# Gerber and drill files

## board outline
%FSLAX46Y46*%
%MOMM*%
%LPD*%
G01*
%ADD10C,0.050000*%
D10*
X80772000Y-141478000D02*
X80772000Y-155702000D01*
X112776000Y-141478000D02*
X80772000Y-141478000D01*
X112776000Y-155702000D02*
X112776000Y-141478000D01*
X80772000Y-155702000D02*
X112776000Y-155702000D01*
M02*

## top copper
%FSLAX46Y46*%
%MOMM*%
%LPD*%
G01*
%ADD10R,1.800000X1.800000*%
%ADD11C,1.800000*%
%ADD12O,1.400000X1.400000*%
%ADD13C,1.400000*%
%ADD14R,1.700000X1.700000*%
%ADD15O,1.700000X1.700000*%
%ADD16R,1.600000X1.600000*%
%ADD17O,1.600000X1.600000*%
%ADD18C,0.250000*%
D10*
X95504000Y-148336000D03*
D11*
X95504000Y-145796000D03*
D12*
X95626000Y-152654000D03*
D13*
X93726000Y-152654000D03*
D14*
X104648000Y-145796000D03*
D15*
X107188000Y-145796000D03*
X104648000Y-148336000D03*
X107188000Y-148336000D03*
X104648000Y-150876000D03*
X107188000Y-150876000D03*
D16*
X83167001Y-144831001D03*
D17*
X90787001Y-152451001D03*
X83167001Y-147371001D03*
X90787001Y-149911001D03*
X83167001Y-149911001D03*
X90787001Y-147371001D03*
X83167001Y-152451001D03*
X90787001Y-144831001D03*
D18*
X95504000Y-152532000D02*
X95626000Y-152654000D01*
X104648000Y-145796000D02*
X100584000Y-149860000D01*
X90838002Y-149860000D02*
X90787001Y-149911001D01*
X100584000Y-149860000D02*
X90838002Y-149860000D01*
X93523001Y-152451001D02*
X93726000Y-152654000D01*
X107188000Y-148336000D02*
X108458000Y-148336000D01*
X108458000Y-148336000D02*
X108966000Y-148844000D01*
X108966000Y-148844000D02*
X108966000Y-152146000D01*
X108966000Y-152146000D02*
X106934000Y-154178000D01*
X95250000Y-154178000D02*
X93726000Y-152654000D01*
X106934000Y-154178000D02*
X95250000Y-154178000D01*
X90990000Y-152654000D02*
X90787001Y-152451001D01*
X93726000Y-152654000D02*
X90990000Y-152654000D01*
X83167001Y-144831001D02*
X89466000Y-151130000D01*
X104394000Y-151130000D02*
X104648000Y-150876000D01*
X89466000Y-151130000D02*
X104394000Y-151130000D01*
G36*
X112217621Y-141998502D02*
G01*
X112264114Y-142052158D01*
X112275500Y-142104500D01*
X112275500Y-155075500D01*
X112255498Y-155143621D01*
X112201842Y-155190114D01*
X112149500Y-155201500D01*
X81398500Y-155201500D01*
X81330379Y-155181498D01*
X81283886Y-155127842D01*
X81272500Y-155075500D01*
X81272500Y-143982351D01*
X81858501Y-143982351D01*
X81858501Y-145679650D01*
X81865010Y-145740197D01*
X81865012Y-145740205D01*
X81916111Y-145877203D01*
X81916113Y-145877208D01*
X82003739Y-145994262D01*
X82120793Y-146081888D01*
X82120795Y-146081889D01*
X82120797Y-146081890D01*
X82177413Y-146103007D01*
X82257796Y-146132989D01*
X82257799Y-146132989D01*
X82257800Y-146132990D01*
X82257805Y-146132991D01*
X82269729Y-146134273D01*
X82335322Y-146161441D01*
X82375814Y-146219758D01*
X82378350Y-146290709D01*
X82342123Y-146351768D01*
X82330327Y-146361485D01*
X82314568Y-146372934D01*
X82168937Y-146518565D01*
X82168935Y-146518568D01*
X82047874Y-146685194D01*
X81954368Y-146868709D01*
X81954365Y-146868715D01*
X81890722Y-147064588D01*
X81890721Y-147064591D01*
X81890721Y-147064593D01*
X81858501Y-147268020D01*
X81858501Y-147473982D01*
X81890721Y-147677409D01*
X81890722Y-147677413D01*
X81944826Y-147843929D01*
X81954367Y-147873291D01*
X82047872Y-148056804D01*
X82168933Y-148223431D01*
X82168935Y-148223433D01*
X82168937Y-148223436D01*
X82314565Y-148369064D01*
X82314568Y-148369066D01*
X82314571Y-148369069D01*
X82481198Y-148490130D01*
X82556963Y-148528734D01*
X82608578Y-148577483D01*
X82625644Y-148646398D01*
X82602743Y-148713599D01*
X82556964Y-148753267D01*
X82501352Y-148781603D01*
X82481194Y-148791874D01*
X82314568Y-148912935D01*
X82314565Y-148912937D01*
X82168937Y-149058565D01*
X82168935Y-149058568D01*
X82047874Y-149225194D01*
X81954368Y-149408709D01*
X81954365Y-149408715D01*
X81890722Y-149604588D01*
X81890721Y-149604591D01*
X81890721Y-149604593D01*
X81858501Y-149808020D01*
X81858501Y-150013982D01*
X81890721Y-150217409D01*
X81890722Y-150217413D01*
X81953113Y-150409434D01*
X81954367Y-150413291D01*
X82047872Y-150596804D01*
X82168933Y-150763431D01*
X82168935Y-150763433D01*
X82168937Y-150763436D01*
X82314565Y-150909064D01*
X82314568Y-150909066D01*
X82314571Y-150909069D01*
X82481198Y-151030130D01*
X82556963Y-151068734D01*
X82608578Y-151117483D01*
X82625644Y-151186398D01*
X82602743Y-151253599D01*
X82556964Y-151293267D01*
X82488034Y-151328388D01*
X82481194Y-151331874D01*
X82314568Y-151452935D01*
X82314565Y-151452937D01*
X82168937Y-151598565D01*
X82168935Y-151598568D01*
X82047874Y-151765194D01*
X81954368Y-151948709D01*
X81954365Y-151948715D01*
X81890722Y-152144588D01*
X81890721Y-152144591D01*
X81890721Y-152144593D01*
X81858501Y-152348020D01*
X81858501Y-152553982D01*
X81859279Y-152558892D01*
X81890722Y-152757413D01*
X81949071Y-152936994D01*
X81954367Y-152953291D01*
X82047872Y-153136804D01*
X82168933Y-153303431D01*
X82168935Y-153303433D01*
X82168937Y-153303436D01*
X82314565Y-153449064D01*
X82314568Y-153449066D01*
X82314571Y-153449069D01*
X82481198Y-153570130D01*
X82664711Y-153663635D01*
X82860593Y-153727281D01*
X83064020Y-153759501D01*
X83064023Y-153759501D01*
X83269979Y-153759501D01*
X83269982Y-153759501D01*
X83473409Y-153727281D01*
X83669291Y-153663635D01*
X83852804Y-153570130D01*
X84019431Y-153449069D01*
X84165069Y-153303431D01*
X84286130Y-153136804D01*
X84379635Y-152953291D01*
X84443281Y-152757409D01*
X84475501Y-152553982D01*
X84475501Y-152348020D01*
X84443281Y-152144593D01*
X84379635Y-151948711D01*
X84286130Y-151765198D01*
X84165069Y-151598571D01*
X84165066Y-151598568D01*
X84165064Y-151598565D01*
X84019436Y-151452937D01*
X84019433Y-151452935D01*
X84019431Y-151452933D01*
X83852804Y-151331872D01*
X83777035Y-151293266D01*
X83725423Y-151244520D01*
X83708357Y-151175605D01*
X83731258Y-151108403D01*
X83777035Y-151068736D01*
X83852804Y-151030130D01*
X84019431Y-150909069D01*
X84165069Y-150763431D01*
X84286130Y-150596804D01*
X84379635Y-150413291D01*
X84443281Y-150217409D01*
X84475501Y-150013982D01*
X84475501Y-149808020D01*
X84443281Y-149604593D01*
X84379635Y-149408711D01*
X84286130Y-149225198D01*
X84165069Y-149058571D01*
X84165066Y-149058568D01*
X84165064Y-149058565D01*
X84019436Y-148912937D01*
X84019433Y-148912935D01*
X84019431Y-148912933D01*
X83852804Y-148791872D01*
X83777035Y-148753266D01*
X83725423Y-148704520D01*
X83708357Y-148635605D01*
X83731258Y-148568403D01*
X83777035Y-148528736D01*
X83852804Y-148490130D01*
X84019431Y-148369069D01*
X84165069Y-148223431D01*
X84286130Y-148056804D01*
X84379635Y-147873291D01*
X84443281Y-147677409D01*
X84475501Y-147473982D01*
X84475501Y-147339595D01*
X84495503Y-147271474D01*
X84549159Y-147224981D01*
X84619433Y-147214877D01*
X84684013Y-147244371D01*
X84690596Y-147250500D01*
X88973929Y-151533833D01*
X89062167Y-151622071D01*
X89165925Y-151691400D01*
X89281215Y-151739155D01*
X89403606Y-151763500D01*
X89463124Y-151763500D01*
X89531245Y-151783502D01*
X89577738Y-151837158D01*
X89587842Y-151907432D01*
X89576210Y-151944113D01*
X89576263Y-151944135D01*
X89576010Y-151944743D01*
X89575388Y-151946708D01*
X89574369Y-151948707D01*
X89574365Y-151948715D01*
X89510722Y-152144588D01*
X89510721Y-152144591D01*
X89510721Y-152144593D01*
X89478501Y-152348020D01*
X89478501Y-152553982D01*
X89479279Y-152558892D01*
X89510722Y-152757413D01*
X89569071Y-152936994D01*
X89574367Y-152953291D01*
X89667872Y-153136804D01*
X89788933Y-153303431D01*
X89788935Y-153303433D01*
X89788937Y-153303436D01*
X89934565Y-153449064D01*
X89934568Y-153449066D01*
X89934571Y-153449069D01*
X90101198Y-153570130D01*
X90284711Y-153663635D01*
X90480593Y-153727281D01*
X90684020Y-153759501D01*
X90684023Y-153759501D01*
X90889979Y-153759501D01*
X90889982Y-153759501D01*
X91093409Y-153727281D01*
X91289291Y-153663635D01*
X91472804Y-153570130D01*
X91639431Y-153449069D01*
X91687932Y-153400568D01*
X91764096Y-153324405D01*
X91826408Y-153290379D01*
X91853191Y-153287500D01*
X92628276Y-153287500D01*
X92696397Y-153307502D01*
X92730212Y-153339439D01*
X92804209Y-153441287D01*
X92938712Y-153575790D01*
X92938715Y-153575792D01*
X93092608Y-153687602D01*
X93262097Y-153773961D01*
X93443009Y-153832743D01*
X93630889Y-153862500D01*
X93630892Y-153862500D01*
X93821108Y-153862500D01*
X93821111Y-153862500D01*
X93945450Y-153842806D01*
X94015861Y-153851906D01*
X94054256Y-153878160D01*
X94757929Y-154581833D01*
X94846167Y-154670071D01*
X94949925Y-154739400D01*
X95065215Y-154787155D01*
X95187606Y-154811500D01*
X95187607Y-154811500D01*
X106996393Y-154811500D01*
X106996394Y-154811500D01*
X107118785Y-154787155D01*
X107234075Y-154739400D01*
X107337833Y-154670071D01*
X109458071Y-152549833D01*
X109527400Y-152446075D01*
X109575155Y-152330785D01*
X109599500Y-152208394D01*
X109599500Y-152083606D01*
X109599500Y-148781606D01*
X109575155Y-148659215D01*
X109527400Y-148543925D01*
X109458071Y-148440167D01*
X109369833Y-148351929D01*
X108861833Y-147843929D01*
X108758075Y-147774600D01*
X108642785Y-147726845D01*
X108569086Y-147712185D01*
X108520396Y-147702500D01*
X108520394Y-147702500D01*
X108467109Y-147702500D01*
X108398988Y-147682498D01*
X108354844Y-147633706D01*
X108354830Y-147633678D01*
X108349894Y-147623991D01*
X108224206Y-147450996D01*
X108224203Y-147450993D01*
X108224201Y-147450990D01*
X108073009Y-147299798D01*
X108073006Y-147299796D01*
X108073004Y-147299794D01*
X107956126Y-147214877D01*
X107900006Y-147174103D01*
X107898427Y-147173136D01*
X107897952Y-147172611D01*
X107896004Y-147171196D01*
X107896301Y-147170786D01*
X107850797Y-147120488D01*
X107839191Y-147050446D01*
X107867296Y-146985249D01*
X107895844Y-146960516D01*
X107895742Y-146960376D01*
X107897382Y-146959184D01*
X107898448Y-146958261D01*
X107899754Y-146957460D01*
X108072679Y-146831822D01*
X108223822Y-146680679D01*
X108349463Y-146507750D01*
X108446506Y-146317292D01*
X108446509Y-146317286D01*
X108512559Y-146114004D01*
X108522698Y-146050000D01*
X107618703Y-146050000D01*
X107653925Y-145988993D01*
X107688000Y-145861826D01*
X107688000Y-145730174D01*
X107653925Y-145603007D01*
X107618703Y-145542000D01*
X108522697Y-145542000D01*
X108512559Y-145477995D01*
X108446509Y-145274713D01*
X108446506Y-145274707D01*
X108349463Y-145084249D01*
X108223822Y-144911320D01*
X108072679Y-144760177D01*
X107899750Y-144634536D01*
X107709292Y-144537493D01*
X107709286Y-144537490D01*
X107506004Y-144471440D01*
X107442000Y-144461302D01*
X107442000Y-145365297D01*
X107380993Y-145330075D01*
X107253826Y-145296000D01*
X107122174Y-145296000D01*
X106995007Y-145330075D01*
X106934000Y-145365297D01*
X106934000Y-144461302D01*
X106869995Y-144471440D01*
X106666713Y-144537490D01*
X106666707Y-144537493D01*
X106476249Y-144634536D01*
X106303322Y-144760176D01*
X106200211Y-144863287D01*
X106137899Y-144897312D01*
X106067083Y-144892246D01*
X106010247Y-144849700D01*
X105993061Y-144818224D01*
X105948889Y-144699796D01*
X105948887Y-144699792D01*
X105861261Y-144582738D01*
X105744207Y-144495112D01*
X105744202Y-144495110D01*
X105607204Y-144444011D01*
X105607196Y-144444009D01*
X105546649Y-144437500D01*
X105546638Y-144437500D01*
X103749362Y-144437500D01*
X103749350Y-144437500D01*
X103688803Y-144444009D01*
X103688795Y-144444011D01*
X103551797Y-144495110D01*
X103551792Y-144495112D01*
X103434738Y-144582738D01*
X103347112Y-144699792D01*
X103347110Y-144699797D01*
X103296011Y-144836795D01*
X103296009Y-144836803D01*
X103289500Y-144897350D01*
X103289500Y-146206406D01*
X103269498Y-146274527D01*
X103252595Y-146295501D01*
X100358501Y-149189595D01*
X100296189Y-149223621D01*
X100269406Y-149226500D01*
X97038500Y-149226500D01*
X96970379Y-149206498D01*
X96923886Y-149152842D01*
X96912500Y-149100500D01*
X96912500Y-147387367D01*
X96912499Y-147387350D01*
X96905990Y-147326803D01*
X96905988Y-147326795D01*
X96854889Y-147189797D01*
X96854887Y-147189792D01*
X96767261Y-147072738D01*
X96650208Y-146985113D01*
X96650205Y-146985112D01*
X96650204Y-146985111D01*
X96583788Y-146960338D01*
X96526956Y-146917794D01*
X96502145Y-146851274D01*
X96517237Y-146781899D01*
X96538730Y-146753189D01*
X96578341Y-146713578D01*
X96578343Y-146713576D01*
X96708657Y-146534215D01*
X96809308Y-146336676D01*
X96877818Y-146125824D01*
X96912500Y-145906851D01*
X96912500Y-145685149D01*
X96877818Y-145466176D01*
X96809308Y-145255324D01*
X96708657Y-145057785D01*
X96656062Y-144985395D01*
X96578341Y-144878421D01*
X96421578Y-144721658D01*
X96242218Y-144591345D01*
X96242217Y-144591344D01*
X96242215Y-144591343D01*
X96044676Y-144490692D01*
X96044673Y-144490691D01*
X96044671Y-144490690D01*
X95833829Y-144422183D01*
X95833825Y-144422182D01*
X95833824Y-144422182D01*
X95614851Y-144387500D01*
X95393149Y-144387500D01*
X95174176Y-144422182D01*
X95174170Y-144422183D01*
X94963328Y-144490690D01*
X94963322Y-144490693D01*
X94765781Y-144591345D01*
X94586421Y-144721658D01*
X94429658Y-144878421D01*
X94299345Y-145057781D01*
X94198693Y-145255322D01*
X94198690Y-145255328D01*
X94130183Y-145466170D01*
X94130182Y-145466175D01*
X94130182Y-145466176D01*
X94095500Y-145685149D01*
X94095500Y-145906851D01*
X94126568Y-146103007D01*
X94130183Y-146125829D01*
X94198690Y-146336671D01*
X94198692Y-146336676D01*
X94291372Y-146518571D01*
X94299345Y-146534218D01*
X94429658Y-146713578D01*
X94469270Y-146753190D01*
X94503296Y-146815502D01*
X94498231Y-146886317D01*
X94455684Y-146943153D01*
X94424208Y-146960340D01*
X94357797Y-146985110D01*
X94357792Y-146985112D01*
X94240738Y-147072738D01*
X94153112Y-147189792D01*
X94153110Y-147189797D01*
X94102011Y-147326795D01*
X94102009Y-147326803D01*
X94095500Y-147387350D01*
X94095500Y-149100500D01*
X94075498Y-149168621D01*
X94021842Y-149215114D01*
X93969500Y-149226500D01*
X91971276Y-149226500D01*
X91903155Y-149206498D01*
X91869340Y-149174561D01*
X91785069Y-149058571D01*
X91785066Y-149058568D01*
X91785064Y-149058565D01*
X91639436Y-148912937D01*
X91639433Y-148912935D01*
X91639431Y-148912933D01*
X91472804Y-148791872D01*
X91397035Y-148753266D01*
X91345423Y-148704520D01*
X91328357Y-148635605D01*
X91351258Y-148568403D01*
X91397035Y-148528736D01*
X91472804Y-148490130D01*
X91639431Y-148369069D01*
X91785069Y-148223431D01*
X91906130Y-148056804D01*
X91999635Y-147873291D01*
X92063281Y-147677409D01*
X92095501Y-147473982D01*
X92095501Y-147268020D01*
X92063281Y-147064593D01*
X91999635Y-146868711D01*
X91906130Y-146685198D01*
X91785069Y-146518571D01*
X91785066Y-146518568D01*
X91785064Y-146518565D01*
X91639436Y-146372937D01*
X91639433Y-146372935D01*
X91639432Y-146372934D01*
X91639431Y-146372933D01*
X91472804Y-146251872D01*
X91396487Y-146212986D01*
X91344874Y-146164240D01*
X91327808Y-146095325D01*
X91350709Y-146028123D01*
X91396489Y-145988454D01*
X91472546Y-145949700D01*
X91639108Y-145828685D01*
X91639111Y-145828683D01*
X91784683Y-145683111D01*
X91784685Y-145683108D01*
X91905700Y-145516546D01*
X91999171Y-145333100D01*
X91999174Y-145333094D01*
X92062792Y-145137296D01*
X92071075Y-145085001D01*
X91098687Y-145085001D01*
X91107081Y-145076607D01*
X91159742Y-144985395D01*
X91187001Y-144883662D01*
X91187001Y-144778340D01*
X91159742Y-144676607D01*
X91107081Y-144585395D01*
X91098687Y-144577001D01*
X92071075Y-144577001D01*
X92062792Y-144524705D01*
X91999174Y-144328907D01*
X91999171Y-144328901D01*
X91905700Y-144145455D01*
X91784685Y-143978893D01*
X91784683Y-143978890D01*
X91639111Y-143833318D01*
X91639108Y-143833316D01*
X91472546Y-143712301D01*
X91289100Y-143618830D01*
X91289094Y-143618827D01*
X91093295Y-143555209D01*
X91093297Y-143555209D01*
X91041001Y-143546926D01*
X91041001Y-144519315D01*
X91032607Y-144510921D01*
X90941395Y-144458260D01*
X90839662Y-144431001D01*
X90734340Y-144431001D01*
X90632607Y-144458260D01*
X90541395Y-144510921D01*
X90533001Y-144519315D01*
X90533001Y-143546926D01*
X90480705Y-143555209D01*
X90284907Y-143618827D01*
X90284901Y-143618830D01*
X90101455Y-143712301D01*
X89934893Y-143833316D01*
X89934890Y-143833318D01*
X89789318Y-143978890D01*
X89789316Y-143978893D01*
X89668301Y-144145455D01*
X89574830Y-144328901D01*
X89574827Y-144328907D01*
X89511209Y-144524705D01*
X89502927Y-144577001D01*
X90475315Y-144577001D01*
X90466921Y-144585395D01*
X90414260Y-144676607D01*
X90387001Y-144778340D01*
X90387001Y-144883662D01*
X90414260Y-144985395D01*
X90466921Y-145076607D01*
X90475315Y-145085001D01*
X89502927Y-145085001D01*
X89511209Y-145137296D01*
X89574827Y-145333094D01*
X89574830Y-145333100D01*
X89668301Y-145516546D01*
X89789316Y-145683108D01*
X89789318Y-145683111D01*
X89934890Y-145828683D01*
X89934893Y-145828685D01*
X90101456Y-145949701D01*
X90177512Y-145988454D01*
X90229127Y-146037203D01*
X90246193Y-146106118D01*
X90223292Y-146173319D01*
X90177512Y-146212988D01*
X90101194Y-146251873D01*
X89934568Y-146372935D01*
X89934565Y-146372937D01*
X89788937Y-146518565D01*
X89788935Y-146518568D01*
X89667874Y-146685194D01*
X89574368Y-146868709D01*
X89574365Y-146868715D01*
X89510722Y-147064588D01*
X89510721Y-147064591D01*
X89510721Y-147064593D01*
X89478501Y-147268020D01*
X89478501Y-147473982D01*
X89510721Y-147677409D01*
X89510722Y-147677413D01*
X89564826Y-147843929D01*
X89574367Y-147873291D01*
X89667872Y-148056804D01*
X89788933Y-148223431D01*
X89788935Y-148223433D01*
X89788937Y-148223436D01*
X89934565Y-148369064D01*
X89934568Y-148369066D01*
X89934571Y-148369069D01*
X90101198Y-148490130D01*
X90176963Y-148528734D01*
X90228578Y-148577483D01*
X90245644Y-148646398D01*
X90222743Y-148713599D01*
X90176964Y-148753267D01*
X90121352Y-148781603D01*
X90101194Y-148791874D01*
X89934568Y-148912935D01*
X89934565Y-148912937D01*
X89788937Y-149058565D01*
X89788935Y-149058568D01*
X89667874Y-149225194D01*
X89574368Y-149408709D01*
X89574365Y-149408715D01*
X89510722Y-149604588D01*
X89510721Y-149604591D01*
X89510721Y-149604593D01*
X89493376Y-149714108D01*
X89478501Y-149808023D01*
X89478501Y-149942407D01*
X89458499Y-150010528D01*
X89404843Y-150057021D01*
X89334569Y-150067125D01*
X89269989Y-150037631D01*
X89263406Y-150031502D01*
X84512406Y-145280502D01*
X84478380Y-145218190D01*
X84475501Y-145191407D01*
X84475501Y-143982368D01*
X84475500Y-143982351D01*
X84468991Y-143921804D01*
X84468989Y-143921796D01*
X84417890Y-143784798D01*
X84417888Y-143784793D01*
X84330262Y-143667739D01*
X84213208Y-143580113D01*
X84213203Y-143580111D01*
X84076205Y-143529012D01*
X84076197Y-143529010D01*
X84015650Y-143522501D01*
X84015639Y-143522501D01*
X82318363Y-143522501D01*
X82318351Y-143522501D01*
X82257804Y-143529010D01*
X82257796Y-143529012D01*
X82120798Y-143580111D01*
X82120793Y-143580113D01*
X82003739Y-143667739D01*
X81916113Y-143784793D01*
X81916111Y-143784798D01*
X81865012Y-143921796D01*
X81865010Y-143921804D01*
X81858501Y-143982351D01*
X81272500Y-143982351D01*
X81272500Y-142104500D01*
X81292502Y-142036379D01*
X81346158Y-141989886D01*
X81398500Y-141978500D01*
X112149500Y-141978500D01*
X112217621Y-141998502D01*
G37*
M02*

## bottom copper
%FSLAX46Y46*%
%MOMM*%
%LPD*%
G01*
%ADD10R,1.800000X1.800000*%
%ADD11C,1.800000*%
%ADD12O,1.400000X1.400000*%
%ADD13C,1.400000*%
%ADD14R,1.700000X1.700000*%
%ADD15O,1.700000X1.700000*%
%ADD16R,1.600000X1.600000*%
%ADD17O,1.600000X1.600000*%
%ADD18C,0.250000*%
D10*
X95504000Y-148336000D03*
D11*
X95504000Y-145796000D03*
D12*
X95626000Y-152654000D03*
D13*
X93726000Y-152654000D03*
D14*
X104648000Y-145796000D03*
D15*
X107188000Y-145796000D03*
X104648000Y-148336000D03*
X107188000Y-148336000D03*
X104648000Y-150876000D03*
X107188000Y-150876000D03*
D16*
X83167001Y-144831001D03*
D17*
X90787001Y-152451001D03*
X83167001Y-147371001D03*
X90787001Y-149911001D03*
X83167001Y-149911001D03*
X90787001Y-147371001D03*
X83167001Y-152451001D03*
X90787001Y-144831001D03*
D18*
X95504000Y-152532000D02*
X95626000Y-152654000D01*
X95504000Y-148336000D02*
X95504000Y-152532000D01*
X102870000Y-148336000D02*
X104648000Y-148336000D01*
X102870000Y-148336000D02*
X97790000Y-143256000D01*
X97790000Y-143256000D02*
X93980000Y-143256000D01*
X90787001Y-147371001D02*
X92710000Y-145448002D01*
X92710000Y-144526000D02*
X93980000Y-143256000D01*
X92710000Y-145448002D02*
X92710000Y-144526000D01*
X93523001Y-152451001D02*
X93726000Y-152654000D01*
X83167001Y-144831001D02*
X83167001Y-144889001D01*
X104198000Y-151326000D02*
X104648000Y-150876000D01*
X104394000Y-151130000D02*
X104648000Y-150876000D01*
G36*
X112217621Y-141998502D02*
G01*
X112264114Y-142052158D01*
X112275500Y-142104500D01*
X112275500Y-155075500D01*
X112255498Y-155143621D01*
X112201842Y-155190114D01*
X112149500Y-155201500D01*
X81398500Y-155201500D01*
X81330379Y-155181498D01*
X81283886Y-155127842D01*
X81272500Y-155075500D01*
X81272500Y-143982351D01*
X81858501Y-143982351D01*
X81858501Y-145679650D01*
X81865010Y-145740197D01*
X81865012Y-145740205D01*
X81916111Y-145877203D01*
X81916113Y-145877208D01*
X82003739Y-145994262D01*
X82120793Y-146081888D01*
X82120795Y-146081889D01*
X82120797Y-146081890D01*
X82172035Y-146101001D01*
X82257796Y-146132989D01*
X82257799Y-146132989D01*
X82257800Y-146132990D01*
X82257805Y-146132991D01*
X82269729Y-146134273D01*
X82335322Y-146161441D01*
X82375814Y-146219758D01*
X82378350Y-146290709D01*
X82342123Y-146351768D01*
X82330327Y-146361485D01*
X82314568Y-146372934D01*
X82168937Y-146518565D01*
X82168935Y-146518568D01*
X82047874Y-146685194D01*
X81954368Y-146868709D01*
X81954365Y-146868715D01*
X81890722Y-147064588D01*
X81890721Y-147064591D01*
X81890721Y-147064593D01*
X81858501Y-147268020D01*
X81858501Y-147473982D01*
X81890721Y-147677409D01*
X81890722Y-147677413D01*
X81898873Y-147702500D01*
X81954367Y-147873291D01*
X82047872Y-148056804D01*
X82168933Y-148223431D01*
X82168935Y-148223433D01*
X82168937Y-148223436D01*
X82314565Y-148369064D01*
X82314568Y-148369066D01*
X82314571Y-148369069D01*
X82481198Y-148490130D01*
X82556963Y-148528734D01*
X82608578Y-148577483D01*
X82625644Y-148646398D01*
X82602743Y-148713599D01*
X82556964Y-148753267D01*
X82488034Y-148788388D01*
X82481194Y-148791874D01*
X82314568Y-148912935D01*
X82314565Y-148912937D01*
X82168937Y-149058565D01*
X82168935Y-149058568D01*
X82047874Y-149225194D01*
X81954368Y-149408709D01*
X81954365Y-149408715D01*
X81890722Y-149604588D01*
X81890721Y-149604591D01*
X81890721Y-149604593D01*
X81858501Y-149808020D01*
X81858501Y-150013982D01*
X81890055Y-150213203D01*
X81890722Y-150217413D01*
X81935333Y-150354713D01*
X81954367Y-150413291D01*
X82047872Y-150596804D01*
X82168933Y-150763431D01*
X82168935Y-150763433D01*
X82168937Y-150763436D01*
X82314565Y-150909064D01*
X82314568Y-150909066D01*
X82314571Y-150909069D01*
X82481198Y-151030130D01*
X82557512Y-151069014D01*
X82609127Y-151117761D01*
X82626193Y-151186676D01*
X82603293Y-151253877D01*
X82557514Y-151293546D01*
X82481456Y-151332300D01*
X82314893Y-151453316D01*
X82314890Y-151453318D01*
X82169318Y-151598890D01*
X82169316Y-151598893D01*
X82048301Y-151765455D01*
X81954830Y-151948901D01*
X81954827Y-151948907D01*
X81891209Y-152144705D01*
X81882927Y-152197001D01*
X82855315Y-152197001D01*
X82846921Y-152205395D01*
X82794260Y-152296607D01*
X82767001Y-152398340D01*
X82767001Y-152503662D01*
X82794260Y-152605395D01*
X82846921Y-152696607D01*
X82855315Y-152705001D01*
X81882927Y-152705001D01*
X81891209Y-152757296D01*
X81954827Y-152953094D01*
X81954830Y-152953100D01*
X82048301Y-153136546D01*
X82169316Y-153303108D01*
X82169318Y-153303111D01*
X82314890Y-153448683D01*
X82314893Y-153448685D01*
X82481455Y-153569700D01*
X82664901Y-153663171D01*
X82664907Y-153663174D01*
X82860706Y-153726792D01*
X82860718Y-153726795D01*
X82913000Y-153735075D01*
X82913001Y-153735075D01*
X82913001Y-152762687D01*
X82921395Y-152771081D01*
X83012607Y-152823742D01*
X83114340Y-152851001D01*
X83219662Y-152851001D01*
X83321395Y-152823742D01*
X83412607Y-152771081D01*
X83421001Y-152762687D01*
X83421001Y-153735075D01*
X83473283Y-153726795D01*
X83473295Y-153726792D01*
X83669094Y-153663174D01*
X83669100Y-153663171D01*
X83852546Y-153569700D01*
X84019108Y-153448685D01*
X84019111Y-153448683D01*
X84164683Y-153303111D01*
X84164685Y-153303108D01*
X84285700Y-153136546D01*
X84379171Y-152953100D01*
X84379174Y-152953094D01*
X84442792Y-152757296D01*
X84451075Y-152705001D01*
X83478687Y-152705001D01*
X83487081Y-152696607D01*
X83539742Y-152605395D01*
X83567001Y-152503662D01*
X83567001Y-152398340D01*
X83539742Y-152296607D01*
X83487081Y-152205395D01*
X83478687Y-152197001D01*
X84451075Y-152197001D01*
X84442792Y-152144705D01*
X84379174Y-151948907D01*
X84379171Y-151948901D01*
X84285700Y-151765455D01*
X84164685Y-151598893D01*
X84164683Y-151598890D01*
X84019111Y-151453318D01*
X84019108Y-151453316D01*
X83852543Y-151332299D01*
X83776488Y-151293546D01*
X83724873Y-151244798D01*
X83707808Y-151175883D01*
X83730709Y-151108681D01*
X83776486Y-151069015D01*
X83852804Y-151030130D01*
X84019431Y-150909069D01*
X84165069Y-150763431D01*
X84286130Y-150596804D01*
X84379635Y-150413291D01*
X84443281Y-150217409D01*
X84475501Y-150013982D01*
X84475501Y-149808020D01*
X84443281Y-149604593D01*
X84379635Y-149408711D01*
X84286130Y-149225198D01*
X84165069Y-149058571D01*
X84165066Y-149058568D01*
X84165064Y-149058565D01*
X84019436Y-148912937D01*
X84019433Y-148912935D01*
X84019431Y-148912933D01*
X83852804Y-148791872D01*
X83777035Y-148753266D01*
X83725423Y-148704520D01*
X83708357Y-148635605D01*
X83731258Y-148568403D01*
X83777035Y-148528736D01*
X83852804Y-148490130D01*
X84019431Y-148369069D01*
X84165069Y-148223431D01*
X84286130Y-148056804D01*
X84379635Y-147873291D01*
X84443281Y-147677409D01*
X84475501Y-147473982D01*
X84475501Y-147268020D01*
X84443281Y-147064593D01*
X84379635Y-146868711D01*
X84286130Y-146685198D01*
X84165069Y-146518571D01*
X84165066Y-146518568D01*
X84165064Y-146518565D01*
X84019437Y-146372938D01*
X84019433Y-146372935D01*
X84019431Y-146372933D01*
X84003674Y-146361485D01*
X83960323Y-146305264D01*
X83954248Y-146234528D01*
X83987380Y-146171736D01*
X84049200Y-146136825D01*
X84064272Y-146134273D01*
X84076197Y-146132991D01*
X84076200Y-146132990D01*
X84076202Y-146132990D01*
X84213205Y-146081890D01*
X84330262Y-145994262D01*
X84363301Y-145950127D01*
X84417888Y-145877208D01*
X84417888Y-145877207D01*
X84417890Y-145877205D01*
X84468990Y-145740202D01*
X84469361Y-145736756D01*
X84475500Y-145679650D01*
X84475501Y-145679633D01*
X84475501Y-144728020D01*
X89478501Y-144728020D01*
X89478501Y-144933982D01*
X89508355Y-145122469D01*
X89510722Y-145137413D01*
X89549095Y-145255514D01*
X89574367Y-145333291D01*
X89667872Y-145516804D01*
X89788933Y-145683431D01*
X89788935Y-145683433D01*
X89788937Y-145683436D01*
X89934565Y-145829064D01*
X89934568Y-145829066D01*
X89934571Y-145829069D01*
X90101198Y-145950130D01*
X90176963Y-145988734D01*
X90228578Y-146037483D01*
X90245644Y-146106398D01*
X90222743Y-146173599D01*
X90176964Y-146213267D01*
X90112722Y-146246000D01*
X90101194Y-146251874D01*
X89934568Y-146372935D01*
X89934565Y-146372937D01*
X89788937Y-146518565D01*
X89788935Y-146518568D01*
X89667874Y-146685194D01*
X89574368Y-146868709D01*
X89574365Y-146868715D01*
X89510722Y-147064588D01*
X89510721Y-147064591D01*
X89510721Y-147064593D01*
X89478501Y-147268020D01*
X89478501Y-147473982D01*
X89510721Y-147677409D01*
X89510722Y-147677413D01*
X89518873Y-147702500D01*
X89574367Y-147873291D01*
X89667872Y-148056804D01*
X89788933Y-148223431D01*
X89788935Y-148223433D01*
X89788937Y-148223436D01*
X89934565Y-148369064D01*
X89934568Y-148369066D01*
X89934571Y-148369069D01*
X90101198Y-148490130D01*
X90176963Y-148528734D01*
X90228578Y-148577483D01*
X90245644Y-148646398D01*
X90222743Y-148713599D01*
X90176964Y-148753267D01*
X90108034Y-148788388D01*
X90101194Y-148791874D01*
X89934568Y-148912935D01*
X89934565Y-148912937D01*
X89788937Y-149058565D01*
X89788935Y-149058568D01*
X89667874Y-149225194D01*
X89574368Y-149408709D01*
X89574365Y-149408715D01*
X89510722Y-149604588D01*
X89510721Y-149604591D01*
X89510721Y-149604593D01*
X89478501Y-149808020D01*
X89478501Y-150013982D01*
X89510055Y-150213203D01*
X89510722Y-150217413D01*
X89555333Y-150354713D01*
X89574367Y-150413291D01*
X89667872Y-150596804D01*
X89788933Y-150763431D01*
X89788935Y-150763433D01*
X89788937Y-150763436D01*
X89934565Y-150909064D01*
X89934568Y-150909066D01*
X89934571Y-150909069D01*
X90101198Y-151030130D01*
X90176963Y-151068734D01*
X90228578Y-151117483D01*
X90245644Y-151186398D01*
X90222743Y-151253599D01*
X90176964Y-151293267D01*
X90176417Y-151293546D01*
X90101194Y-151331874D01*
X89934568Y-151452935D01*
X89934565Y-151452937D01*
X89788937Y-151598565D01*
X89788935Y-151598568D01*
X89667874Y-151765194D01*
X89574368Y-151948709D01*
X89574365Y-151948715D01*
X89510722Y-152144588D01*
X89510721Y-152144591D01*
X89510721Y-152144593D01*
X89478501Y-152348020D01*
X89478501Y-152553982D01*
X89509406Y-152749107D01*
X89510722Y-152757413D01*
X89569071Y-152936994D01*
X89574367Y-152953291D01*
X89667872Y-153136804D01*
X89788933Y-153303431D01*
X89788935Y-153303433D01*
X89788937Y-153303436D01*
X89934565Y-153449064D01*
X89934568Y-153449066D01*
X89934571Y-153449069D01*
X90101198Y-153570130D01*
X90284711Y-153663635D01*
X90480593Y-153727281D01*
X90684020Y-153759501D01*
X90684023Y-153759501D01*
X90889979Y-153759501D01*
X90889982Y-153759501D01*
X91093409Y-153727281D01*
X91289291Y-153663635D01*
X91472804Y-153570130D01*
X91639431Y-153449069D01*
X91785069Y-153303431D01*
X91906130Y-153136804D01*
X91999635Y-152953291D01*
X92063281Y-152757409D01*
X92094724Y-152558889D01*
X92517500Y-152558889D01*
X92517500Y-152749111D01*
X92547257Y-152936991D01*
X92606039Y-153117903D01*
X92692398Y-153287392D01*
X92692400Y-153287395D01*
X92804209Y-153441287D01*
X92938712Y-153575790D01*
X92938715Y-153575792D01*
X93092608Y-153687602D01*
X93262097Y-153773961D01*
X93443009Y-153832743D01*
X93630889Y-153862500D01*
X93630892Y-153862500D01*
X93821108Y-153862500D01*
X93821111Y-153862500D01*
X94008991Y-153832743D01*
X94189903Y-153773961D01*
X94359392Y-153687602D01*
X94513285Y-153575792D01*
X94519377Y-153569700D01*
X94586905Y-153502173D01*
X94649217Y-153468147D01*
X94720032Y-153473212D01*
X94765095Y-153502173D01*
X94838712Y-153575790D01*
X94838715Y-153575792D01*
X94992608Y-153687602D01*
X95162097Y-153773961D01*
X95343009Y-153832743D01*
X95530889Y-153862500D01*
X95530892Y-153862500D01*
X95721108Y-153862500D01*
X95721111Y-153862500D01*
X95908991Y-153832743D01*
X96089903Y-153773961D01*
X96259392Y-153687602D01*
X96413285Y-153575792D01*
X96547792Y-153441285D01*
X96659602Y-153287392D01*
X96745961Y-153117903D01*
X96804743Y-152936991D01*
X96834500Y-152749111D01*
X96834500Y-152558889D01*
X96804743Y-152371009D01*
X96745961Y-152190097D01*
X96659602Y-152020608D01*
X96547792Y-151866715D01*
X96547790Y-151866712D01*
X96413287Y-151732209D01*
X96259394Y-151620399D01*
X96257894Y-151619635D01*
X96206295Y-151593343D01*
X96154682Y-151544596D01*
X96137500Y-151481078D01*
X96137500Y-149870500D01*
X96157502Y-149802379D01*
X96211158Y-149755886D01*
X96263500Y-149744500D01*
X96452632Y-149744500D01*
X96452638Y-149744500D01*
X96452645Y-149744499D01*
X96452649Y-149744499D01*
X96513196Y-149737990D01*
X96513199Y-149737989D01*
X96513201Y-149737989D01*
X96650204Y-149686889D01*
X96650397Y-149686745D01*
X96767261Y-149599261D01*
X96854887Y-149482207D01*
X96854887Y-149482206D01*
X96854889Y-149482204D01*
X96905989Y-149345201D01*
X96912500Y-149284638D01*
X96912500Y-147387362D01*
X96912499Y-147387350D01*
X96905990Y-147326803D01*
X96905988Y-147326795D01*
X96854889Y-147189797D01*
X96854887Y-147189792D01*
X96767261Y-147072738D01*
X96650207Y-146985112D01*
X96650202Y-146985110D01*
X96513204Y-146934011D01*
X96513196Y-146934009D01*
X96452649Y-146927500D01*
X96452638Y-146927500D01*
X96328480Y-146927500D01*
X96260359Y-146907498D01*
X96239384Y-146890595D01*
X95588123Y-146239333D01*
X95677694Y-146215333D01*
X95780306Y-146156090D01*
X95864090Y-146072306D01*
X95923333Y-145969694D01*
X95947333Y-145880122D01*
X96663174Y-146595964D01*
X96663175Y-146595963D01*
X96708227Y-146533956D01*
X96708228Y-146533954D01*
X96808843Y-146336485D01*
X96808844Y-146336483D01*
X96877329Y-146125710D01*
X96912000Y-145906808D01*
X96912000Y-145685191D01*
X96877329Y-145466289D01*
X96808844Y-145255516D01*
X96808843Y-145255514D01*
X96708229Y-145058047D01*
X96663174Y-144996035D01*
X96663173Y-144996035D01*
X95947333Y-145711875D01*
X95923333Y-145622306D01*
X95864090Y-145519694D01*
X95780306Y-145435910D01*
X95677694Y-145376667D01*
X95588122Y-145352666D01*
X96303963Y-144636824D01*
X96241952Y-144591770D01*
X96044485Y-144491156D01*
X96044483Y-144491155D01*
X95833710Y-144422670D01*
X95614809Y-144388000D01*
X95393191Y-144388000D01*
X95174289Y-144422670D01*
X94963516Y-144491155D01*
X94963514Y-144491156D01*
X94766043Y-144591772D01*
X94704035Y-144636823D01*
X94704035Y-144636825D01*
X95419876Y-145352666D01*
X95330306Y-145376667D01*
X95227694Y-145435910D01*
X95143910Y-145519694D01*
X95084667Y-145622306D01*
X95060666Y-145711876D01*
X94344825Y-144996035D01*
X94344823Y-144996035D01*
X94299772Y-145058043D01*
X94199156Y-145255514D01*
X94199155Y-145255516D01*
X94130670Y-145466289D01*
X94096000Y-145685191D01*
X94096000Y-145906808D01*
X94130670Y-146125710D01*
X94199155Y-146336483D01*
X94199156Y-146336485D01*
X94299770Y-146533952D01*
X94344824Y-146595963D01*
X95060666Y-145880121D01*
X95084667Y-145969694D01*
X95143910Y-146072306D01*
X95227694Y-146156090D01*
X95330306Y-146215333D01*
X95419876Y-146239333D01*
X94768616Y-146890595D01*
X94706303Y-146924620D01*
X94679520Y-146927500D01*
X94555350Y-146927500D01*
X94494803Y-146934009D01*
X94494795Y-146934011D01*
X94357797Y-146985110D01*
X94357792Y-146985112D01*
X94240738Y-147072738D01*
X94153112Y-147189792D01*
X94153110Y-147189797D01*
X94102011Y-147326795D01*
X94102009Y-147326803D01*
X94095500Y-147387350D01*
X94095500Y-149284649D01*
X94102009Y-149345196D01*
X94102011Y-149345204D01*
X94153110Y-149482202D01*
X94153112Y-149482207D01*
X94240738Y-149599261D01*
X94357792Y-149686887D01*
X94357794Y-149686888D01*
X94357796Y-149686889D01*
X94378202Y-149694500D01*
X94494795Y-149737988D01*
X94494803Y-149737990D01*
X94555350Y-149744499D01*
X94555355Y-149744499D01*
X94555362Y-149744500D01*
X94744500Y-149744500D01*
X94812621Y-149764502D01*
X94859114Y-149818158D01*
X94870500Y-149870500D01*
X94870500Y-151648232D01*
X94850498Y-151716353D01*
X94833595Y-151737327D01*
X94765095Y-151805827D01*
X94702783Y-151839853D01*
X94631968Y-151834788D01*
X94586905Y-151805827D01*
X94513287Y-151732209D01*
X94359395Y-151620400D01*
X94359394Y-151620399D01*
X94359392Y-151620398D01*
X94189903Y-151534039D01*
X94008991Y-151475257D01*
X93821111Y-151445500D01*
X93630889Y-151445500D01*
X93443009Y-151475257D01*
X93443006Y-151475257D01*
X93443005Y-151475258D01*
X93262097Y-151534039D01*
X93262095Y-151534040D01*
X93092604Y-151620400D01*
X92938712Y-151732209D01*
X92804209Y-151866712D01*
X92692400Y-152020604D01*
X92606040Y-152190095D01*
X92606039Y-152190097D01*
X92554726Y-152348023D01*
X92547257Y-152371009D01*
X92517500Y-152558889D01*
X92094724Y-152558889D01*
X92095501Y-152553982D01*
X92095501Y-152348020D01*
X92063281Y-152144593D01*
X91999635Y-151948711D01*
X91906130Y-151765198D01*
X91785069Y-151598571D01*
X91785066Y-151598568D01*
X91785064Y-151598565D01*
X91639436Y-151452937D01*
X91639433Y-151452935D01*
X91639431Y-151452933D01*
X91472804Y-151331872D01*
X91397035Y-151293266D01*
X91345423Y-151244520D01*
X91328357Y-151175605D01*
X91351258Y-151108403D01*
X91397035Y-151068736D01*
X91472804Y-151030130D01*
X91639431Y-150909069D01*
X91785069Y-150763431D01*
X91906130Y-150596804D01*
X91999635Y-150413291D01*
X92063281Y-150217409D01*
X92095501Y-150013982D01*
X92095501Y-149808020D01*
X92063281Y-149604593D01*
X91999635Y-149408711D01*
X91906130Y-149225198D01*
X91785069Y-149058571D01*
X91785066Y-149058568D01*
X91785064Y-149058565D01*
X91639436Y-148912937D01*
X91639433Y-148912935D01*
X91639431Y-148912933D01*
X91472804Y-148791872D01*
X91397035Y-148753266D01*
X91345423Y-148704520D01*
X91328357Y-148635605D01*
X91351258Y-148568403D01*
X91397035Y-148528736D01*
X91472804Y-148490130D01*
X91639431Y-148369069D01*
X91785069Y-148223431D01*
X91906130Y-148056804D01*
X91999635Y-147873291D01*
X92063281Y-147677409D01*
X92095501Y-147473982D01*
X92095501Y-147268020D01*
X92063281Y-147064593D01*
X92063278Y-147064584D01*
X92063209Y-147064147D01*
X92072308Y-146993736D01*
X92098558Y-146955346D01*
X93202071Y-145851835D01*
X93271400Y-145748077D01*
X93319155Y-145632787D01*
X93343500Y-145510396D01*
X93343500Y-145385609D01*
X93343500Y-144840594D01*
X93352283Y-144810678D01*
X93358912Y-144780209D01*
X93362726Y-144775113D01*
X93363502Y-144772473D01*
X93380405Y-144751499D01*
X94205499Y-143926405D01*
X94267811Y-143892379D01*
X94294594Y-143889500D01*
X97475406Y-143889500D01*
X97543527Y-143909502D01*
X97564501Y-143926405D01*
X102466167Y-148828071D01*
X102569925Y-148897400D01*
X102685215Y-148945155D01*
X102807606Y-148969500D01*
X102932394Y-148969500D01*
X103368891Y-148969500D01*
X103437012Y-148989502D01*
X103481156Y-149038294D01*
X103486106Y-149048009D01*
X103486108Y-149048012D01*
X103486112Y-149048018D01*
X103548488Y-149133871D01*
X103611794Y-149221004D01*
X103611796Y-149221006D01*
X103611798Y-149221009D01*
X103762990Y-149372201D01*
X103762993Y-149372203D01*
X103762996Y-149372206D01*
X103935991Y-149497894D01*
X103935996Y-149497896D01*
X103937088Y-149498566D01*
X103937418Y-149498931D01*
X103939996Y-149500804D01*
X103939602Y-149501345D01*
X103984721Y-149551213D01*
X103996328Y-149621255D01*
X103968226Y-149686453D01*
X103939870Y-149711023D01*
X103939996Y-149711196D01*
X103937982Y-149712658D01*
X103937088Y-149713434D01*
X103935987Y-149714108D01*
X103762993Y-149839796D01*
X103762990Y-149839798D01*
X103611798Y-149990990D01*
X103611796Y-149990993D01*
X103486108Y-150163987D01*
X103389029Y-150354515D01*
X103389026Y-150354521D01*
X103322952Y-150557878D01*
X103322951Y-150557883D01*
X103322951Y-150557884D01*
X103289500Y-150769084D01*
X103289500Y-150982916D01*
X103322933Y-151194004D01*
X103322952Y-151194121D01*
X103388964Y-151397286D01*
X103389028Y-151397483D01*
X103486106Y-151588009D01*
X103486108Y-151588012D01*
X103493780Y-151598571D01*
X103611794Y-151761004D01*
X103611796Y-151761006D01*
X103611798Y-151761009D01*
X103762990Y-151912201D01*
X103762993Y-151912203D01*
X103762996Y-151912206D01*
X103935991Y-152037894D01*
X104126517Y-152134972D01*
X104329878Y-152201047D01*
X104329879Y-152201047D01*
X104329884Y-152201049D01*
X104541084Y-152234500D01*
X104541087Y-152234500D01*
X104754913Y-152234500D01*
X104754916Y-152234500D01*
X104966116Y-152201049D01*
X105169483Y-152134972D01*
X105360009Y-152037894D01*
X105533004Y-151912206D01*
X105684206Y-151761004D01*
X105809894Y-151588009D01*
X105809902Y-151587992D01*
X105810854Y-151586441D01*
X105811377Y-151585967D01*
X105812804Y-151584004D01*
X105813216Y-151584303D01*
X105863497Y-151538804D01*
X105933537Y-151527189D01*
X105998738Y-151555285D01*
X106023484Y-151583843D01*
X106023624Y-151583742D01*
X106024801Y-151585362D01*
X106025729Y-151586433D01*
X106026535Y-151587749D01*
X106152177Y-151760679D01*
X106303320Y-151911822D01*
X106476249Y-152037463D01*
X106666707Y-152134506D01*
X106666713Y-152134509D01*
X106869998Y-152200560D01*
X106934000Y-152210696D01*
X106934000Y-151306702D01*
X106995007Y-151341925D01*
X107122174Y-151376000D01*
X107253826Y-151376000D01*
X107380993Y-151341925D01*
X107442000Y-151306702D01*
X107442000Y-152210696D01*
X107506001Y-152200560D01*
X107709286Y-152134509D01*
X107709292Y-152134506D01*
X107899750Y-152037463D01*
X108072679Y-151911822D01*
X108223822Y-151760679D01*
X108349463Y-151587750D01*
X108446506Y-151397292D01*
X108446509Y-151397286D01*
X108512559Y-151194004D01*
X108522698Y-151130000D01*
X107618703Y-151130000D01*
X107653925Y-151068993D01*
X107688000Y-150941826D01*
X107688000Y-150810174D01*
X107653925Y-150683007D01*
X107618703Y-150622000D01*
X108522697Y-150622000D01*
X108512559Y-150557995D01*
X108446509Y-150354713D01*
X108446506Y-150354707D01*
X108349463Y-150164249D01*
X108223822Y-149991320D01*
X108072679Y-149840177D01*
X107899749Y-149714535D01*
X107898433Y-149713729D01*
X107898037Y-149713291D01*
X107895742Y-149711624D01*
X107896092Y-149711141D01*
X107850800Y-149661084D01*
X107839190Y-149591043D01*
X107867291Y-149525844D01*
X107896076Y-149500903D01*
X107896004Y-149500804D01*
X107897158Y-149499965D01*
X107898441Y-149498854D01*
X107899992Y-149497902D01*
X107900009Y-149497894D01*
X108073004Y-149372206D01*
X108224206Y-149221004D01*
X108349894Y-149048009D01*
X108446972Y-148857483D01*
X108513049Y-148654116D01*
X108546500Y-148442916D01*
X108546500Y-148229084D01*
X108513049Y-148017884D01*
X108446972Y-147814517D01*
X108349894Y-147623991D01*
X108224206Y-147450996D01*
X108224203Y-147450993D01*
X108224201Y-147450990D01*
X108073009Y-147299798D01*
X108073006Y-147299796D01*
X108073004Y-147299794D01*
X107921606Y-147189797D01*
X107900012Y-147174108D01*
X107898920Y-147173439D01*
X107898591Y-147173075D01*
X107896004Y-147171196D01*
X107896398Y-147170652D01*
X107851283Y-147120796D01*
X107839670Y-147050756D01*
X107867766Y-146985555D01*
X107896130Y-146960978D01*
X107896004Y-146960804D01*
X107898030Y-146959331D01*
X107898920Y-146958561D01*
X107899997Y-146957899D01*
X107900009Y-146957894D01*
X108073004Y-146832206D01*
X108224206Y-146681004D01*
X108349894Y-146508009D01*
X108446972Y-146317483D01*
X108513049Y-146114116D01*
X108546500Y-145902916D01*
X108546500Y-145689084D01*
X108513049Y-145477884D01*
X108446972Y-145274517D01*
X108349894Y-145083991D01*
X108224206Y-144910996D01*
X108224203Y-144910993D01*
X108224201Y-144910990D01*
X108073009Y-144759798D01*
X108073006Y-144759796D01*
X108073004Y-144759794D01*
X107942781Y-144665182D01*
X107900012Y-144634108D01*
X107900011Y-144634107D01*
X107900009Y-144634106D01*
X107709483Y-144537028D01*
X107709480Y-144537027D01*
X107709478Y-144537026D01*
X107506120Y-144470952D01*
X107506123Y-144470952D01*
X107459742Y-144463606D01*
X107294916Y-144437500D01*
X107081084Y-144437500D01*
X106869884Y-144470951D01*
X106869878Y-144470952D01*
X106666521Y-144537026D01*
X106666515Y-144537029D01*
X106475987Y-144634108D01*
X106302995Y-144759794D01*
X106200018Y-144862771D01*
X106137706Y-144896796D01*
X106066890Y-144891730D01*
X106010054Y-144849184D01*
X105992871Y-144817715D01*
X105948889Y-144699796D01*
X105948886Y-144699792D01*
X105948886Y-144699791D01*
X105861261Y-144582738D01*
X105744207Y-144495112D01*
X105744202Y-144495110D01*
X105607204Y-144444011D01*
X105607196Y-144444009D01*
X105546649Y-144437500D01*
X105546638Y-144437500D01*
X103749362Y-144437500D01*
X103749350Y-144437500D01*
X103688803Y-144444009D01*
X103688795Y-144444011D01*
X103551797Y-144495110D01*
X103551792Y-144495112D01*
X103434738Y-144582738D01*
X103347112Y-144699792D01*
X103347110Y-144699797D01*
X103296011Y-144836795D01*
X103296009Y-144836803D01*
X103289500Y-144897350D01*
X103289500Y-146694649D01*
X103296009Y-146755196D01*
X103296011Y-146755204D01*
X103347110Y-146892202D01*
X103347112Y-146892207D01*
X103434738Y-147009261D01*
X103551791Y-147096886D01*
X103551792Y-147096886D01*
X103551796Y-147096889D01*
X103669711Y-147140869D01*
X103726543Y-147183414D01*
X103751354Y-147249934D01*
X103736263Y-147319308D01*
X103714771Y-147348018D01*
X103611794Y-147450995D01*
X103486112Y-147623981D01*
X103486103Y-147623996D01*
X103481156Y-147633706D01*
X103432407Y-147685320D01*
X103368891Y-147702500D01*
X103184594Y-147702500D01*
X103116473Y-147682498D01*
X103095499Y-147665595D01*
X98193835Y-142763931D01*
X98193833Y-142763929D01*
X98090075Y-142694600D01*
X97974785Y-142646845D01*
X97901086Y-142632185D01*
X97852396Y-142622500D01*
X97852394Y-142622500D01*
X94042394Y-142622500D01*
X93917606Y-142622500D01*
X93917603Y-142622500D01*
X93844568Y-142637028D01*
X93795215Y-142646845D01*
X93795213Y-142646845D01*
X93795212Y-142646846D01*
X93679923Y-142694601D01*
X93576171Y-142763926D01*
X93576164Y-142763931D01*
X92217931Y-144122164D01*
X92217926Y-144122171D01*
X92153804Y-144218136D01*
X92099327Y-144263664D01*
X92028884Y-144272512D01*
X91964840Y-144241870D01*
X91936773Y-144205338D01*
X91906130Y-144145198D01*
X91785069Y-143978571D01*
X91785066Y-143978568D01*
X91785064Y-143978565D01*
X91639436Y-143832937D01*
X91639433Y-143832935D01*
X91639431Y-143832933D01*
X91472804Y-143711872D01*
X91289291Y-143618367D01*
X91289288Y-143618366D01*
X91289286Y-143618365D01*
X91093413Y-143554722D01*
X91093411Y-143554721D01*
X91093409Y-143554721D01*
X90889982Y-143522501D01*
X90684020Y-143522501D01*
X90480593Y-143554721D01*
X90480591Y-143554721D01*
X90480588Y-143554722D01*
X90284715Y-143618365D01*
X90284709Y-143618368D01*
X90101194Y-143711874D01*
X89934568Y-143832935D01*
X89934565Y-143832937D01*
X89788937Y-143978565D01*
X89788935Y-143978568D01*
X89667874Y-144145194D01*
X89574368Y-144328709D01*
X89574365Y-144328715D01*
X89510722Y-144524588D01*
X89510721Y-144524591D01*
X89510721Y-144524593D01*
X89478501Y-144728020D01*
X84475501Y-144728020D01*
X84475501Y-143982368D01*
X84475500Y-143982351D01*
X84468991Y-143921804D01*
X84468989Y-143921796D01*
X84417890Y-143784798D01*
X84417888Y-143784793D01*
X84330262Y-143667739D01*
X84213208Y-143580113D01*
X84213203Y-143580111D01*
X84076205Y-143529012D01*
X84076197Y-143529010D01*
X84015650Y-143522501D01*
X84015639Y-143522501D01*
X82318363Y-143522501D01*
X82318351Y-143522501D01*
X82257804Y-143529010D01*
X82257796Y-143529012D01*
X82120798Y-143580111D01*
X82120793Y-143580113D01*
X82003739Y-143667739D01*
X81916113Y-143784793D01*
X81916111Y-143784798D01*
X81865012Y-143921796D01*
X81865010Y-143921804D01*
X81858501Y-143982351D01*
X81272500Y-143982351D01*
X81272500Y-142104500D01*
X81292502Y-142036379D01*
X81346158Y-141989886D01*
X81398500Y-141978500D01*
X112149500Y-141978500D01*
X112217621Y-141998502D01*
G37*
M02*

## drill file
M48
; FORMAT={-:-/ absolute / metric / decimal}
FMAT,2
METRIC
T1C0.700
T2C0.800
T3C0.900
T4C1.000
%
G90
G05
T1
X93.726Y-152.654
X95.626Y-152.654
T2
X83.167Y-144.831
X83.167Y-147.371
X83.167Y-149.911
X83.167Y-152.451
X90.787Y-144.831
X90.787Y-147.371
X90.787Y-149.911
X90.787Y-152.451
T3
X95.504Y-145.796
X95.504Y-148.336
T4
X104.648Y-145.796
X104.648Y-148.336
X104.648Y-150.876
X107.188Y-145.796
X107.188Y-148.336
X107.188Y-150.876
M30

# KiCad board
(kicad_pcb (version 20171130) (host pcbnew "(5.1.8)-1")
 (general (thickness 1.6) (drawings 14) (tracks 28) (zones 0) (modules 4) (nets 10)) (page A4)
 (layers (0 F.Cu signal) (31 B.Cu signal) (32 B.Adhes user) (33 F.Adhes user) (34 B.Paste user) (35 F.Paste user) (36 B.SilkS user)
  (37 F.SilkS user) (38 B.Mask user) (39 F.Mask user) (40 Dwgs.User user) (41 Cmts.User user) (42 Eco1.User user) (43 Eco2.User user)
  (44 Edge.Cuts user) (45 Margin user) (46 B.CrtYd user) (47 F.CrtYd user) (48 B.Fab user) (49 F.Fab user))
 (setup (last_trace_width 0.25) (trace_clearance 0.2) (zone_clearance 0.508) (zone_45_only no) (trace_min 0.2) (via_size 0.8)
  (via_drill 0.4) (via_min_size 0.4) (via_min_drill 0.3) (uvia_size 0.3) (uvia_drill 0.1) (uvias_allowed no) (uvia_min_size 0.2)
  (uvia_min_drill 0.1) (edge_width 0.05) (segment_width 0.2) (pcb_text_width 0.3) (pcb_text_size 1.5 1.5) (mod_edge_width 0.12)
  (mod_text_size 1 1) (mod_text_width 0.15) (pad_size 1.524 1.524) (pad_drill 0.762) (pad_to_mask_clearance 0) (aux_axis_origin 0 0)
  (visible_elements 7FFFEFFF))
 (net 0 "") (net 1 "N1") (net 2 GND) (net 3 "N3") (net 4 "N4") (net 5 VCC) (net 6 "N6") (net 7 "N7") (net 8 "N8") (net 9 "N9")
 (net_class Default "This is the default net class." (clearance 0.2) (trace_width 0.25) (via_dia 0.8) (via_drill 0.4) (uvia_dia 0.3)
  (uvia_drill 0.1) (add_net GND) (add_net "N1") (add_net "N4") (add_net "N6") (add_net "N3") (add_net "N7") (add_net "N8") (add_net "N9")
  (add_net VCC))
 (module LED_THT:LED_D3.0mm (layer F.Cu) (at 95.504 148.336 90)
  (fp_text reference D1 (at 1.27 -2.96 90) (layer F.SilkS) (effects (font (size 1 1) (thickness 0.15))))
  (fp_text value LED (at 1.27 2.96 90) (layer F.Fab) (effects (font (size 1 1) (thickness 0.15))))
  (pad 1 thru_hole rect (at 0 0 90) (size 1.8 1.8) (drill 0.9) (layers *.Cu *.Mask) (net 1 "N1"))
  (pad 2 thru_hole circle (at 2.54 0 90) (size 1.8 1.8) (drill 0.9) (layers *.Cu *.Mask) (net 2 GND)))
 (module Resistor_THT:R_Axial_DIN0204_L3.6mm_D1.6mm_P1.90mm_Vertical (layer F.Cu) (at 93.726 152.654)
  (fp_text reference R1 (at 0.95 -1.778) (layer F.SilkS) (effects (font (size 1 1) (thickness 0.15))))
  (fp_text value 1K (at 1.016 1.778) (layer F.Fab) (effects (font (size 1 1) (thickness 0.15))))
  (pad 2 thru_hole oval (at 1.9 0) (size 1.4 1.4) (drill 0.7) (layers *.Cu *.Mask) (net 1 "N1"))
  (pad 1 thru_hole circle (at 0 0) (size 1.4 1.4) (drill 0.7) (layers *.Cu *.Mask) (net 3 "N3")))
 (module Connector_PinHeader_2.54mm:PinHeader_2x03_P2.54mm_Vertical (layer F.Cu) (at 104.648 145.796)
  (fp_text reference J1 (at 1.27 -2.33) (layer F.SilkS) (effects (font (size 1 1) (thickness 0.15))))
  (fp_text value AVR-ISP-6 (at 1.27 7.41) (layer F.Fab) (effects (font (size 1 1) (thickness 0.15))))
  (pad 1 thru_hole rect (at 0 0) (size 1.7 1.7) (drill 1) (layers *.Cu *.Mask) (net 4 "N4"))
  (pad 2 thru_hole oval (at 2.54 0) (size 1.7 1.7) (drill 1) (layers *.Cu *.Mask) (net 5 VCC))
  (pad 3 thru_hole oval (at 0 2.54) (size 1.7 1.7) (drill 1) (layers *.Cu *.Mask) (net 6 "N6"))
  (pad 4 thru_hole oval (at 2.54 2.54) (size 1.7 1.7) (drill 1) (layers *.Cu *.Mask) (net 3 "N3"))
  (pad 5 thru_hole oval (at 0 5.08) (size 1.7 1.7) (drill 1) (layers *.Cu *.Mask) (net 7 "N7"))
  (pad 6 thru_hole oval (at 2.54 5.08) (size 1.7 1.7) (drill 1) (layers *.Cu *.Mask) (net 2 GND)))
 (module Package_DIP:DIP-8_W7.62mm (layer F.Cu) (at 83.167001 144.831001)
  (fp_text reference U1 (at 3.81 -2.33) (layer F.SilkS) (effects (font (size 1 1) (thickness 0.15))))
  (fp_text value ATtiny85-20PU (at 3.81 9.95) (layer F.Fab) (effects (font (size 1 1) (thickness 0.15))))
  (pad 1 thru_hole rect (at 0 0) (size 1.6 1.6) (drill 0.8) (layers *.Cu *.Mask) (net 7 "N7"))
  (pad 5 thru_hole oval (at 7.62 7.62) (size 1.6 1.6) (drill 0.8) (layers *.Cu *.Mask) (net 3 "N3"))
  (pad 2 thru_hole oval (at 0 2.54) (size 1.6 1.6) (drill 0.8) (layers *.Cu *.Mask) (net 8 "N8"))
  (pad 6 thru_hole oval (at 7.62 5.08) (size 1.6 1.6) (drill 0.8) (layers *.Cu *.Mask) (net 4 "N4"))
  (pad 3 thru_hole oval (at 0 5.08) (size 1.6 1.6) (drill 0.8) (layers *.Cu *.Mask) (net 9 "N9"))
  (pad 7 thru_hole oval (at 7.62 2.54) (size 1.6 1.6) (drill 0.8) (layers *.Cu *.Mask) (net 6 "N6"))
  (pad 4 thru_hole oval (at 0 7.62) (size 1.6 1.6) (drill 0.8) (layers *.Cu *.Mask) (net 2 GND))
  (pad 8 thru_hole oval (at 7.62 0) (size 1.6 1.6) (drill 0.8) (layers *.Cu *.Mask) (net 5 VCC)))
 (gr_line (start 80.772 141.478) (end 80.772 155.702) (layer Edge.Cuts) (width 0.05))
 (gr_line (start 112.776 141.478) (end 80.772 141.478) (layer Edge.Cuts) (width 0.05))
 (gr_line (start 112.776 155.702) (end 112.776 141.478) (layer Edge.Cuts) (width 0.05))
 (gr_line (start 80.772 155.702) (end 112.776 155.702) (layer Edge.Cuts) (width 0.05))
 (segment (start 95.504 152.532) (end 95.626 152.654) (width 0.25) (layer F.Cu) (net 1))
 (segment (start 95.504 152.532) (end 95.626 152.654) (width 0.25) (layer B.Cu) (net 1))
 (segment (start 95.504 148.336) (end 95.504 152.532) (width 0.25) (layer B.Cu) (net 1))
 (segment (start 104.648 145.796) (end 100.584 149.86) (width 0.25) (layer F.Cu) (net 4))
 (segment (start 90.838002 149.86) (end 90.787001 149.911001) (width 0.25) (layer F.Cu) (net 4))
 (segment (start 100.584 149.86) (end 90.838002 149.86) (width 0.25) (layer F.Cu) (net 4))
 (segment (start 102.87 148.336) (end 104.648 148.336) (width 0.25) (layer B.Cu) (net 6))
 (segment (start 102.87 148.336) (end 97.79 143.256) (width 0.25) (layer B.Cu) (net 6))
 (segment (start 97.79 143.256) (end 93.98 143.256) (width 0.25) (layer B.Cu) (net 6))
 (segment (start 90.787001 147.371001) (end 92.71 145.448002) (width 0.25) (layer B.Cu) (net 6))
 (segment (start 92.71 144.526) (end 93.98 143.256) (width 0.25) (layer B.Cu) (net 6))
 (segment (start 92.71 145.448002) (end 92.71 144.526) (width 0.25) (layer B.Cu) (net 6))
 (segment (start 93.523001 152.451001) (end 93.726 152.654) (width 0.25) (layer F.Cu) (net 3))
 (segment (start 93.523001 152.451001) (end 93.726 152.654) (width 0.25) (layer B.Cu) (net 3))
 (segment (start 107.188 148.336) (end 108.458 148.336) (width 0.25) (layer F.Cu) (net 3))
 (segment (start 108.458 148.336) (end 108.966 148.844) (width 0.25) (layer F.Cu) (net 3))
 (segment (start 108.966 148.844) (end 108.966 152.146) (width 0.25) (layer F.Cu) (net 3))
 (segment (start 108.966 152.146) (end 106.934 154.178) (width 0.25) (layer F.Cu) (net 3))
 (segment (start 95.25 154.178) (end 93.726 152.654) (width 0.25) (layer F.Cu) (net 3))
 (segment (start 106.934 154.178) (end 95.25 154.178) (width 0.25) (layer F.Cu) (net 3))
 (segment (start 90.99 152.654) (end 90.787001 152.451001) (width 0.25) (layer F.Cu) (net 3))
 (segment (start 93.726 152.654) (end 90.99 152.654) (width 0.25) (layer F.Cu) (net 3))
 (segment (start 83.167001 144.831001) (end 83.167001 144.889001) (width 0.25) (layer B.Cu) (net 7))
 (segment (start 104.198 151.326) (end 104.648 150.876) (width 0.25) (layer B.Cu) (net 7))
 (segment (start 104.394 151.13) (end 104.648 150.876) (width 0.25) (layer B.Cu) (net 7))
 (segment (start 83.167001 144.831001) (end 89.466 151.13) (width 0.25) (layer F.Cu) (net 7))
 (segment (start 104.394 151.13) (end 104.648 150.876) (width 0.25) (layer F.Cu) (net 7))
 (segment (start 89.466 151.13) (end 104.394 151.13) (width 0.25) (layer F.Cu) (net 7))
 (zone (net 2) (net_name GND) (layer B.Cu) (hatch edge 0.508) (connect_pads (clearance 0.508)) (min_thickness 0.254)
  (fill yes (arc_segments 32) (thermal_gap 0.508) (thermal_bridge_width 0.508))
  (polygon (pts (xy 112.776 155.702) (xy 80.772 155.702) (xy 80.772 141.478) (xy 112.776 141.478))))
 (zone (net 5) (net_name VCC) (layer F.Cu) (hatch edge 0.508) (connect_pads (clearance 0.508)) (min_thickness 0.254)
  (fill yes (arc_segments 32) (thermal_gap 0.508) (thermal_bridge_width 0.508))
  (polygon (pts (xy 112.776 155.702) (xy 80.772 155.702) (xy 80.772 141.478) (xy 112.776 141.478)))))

